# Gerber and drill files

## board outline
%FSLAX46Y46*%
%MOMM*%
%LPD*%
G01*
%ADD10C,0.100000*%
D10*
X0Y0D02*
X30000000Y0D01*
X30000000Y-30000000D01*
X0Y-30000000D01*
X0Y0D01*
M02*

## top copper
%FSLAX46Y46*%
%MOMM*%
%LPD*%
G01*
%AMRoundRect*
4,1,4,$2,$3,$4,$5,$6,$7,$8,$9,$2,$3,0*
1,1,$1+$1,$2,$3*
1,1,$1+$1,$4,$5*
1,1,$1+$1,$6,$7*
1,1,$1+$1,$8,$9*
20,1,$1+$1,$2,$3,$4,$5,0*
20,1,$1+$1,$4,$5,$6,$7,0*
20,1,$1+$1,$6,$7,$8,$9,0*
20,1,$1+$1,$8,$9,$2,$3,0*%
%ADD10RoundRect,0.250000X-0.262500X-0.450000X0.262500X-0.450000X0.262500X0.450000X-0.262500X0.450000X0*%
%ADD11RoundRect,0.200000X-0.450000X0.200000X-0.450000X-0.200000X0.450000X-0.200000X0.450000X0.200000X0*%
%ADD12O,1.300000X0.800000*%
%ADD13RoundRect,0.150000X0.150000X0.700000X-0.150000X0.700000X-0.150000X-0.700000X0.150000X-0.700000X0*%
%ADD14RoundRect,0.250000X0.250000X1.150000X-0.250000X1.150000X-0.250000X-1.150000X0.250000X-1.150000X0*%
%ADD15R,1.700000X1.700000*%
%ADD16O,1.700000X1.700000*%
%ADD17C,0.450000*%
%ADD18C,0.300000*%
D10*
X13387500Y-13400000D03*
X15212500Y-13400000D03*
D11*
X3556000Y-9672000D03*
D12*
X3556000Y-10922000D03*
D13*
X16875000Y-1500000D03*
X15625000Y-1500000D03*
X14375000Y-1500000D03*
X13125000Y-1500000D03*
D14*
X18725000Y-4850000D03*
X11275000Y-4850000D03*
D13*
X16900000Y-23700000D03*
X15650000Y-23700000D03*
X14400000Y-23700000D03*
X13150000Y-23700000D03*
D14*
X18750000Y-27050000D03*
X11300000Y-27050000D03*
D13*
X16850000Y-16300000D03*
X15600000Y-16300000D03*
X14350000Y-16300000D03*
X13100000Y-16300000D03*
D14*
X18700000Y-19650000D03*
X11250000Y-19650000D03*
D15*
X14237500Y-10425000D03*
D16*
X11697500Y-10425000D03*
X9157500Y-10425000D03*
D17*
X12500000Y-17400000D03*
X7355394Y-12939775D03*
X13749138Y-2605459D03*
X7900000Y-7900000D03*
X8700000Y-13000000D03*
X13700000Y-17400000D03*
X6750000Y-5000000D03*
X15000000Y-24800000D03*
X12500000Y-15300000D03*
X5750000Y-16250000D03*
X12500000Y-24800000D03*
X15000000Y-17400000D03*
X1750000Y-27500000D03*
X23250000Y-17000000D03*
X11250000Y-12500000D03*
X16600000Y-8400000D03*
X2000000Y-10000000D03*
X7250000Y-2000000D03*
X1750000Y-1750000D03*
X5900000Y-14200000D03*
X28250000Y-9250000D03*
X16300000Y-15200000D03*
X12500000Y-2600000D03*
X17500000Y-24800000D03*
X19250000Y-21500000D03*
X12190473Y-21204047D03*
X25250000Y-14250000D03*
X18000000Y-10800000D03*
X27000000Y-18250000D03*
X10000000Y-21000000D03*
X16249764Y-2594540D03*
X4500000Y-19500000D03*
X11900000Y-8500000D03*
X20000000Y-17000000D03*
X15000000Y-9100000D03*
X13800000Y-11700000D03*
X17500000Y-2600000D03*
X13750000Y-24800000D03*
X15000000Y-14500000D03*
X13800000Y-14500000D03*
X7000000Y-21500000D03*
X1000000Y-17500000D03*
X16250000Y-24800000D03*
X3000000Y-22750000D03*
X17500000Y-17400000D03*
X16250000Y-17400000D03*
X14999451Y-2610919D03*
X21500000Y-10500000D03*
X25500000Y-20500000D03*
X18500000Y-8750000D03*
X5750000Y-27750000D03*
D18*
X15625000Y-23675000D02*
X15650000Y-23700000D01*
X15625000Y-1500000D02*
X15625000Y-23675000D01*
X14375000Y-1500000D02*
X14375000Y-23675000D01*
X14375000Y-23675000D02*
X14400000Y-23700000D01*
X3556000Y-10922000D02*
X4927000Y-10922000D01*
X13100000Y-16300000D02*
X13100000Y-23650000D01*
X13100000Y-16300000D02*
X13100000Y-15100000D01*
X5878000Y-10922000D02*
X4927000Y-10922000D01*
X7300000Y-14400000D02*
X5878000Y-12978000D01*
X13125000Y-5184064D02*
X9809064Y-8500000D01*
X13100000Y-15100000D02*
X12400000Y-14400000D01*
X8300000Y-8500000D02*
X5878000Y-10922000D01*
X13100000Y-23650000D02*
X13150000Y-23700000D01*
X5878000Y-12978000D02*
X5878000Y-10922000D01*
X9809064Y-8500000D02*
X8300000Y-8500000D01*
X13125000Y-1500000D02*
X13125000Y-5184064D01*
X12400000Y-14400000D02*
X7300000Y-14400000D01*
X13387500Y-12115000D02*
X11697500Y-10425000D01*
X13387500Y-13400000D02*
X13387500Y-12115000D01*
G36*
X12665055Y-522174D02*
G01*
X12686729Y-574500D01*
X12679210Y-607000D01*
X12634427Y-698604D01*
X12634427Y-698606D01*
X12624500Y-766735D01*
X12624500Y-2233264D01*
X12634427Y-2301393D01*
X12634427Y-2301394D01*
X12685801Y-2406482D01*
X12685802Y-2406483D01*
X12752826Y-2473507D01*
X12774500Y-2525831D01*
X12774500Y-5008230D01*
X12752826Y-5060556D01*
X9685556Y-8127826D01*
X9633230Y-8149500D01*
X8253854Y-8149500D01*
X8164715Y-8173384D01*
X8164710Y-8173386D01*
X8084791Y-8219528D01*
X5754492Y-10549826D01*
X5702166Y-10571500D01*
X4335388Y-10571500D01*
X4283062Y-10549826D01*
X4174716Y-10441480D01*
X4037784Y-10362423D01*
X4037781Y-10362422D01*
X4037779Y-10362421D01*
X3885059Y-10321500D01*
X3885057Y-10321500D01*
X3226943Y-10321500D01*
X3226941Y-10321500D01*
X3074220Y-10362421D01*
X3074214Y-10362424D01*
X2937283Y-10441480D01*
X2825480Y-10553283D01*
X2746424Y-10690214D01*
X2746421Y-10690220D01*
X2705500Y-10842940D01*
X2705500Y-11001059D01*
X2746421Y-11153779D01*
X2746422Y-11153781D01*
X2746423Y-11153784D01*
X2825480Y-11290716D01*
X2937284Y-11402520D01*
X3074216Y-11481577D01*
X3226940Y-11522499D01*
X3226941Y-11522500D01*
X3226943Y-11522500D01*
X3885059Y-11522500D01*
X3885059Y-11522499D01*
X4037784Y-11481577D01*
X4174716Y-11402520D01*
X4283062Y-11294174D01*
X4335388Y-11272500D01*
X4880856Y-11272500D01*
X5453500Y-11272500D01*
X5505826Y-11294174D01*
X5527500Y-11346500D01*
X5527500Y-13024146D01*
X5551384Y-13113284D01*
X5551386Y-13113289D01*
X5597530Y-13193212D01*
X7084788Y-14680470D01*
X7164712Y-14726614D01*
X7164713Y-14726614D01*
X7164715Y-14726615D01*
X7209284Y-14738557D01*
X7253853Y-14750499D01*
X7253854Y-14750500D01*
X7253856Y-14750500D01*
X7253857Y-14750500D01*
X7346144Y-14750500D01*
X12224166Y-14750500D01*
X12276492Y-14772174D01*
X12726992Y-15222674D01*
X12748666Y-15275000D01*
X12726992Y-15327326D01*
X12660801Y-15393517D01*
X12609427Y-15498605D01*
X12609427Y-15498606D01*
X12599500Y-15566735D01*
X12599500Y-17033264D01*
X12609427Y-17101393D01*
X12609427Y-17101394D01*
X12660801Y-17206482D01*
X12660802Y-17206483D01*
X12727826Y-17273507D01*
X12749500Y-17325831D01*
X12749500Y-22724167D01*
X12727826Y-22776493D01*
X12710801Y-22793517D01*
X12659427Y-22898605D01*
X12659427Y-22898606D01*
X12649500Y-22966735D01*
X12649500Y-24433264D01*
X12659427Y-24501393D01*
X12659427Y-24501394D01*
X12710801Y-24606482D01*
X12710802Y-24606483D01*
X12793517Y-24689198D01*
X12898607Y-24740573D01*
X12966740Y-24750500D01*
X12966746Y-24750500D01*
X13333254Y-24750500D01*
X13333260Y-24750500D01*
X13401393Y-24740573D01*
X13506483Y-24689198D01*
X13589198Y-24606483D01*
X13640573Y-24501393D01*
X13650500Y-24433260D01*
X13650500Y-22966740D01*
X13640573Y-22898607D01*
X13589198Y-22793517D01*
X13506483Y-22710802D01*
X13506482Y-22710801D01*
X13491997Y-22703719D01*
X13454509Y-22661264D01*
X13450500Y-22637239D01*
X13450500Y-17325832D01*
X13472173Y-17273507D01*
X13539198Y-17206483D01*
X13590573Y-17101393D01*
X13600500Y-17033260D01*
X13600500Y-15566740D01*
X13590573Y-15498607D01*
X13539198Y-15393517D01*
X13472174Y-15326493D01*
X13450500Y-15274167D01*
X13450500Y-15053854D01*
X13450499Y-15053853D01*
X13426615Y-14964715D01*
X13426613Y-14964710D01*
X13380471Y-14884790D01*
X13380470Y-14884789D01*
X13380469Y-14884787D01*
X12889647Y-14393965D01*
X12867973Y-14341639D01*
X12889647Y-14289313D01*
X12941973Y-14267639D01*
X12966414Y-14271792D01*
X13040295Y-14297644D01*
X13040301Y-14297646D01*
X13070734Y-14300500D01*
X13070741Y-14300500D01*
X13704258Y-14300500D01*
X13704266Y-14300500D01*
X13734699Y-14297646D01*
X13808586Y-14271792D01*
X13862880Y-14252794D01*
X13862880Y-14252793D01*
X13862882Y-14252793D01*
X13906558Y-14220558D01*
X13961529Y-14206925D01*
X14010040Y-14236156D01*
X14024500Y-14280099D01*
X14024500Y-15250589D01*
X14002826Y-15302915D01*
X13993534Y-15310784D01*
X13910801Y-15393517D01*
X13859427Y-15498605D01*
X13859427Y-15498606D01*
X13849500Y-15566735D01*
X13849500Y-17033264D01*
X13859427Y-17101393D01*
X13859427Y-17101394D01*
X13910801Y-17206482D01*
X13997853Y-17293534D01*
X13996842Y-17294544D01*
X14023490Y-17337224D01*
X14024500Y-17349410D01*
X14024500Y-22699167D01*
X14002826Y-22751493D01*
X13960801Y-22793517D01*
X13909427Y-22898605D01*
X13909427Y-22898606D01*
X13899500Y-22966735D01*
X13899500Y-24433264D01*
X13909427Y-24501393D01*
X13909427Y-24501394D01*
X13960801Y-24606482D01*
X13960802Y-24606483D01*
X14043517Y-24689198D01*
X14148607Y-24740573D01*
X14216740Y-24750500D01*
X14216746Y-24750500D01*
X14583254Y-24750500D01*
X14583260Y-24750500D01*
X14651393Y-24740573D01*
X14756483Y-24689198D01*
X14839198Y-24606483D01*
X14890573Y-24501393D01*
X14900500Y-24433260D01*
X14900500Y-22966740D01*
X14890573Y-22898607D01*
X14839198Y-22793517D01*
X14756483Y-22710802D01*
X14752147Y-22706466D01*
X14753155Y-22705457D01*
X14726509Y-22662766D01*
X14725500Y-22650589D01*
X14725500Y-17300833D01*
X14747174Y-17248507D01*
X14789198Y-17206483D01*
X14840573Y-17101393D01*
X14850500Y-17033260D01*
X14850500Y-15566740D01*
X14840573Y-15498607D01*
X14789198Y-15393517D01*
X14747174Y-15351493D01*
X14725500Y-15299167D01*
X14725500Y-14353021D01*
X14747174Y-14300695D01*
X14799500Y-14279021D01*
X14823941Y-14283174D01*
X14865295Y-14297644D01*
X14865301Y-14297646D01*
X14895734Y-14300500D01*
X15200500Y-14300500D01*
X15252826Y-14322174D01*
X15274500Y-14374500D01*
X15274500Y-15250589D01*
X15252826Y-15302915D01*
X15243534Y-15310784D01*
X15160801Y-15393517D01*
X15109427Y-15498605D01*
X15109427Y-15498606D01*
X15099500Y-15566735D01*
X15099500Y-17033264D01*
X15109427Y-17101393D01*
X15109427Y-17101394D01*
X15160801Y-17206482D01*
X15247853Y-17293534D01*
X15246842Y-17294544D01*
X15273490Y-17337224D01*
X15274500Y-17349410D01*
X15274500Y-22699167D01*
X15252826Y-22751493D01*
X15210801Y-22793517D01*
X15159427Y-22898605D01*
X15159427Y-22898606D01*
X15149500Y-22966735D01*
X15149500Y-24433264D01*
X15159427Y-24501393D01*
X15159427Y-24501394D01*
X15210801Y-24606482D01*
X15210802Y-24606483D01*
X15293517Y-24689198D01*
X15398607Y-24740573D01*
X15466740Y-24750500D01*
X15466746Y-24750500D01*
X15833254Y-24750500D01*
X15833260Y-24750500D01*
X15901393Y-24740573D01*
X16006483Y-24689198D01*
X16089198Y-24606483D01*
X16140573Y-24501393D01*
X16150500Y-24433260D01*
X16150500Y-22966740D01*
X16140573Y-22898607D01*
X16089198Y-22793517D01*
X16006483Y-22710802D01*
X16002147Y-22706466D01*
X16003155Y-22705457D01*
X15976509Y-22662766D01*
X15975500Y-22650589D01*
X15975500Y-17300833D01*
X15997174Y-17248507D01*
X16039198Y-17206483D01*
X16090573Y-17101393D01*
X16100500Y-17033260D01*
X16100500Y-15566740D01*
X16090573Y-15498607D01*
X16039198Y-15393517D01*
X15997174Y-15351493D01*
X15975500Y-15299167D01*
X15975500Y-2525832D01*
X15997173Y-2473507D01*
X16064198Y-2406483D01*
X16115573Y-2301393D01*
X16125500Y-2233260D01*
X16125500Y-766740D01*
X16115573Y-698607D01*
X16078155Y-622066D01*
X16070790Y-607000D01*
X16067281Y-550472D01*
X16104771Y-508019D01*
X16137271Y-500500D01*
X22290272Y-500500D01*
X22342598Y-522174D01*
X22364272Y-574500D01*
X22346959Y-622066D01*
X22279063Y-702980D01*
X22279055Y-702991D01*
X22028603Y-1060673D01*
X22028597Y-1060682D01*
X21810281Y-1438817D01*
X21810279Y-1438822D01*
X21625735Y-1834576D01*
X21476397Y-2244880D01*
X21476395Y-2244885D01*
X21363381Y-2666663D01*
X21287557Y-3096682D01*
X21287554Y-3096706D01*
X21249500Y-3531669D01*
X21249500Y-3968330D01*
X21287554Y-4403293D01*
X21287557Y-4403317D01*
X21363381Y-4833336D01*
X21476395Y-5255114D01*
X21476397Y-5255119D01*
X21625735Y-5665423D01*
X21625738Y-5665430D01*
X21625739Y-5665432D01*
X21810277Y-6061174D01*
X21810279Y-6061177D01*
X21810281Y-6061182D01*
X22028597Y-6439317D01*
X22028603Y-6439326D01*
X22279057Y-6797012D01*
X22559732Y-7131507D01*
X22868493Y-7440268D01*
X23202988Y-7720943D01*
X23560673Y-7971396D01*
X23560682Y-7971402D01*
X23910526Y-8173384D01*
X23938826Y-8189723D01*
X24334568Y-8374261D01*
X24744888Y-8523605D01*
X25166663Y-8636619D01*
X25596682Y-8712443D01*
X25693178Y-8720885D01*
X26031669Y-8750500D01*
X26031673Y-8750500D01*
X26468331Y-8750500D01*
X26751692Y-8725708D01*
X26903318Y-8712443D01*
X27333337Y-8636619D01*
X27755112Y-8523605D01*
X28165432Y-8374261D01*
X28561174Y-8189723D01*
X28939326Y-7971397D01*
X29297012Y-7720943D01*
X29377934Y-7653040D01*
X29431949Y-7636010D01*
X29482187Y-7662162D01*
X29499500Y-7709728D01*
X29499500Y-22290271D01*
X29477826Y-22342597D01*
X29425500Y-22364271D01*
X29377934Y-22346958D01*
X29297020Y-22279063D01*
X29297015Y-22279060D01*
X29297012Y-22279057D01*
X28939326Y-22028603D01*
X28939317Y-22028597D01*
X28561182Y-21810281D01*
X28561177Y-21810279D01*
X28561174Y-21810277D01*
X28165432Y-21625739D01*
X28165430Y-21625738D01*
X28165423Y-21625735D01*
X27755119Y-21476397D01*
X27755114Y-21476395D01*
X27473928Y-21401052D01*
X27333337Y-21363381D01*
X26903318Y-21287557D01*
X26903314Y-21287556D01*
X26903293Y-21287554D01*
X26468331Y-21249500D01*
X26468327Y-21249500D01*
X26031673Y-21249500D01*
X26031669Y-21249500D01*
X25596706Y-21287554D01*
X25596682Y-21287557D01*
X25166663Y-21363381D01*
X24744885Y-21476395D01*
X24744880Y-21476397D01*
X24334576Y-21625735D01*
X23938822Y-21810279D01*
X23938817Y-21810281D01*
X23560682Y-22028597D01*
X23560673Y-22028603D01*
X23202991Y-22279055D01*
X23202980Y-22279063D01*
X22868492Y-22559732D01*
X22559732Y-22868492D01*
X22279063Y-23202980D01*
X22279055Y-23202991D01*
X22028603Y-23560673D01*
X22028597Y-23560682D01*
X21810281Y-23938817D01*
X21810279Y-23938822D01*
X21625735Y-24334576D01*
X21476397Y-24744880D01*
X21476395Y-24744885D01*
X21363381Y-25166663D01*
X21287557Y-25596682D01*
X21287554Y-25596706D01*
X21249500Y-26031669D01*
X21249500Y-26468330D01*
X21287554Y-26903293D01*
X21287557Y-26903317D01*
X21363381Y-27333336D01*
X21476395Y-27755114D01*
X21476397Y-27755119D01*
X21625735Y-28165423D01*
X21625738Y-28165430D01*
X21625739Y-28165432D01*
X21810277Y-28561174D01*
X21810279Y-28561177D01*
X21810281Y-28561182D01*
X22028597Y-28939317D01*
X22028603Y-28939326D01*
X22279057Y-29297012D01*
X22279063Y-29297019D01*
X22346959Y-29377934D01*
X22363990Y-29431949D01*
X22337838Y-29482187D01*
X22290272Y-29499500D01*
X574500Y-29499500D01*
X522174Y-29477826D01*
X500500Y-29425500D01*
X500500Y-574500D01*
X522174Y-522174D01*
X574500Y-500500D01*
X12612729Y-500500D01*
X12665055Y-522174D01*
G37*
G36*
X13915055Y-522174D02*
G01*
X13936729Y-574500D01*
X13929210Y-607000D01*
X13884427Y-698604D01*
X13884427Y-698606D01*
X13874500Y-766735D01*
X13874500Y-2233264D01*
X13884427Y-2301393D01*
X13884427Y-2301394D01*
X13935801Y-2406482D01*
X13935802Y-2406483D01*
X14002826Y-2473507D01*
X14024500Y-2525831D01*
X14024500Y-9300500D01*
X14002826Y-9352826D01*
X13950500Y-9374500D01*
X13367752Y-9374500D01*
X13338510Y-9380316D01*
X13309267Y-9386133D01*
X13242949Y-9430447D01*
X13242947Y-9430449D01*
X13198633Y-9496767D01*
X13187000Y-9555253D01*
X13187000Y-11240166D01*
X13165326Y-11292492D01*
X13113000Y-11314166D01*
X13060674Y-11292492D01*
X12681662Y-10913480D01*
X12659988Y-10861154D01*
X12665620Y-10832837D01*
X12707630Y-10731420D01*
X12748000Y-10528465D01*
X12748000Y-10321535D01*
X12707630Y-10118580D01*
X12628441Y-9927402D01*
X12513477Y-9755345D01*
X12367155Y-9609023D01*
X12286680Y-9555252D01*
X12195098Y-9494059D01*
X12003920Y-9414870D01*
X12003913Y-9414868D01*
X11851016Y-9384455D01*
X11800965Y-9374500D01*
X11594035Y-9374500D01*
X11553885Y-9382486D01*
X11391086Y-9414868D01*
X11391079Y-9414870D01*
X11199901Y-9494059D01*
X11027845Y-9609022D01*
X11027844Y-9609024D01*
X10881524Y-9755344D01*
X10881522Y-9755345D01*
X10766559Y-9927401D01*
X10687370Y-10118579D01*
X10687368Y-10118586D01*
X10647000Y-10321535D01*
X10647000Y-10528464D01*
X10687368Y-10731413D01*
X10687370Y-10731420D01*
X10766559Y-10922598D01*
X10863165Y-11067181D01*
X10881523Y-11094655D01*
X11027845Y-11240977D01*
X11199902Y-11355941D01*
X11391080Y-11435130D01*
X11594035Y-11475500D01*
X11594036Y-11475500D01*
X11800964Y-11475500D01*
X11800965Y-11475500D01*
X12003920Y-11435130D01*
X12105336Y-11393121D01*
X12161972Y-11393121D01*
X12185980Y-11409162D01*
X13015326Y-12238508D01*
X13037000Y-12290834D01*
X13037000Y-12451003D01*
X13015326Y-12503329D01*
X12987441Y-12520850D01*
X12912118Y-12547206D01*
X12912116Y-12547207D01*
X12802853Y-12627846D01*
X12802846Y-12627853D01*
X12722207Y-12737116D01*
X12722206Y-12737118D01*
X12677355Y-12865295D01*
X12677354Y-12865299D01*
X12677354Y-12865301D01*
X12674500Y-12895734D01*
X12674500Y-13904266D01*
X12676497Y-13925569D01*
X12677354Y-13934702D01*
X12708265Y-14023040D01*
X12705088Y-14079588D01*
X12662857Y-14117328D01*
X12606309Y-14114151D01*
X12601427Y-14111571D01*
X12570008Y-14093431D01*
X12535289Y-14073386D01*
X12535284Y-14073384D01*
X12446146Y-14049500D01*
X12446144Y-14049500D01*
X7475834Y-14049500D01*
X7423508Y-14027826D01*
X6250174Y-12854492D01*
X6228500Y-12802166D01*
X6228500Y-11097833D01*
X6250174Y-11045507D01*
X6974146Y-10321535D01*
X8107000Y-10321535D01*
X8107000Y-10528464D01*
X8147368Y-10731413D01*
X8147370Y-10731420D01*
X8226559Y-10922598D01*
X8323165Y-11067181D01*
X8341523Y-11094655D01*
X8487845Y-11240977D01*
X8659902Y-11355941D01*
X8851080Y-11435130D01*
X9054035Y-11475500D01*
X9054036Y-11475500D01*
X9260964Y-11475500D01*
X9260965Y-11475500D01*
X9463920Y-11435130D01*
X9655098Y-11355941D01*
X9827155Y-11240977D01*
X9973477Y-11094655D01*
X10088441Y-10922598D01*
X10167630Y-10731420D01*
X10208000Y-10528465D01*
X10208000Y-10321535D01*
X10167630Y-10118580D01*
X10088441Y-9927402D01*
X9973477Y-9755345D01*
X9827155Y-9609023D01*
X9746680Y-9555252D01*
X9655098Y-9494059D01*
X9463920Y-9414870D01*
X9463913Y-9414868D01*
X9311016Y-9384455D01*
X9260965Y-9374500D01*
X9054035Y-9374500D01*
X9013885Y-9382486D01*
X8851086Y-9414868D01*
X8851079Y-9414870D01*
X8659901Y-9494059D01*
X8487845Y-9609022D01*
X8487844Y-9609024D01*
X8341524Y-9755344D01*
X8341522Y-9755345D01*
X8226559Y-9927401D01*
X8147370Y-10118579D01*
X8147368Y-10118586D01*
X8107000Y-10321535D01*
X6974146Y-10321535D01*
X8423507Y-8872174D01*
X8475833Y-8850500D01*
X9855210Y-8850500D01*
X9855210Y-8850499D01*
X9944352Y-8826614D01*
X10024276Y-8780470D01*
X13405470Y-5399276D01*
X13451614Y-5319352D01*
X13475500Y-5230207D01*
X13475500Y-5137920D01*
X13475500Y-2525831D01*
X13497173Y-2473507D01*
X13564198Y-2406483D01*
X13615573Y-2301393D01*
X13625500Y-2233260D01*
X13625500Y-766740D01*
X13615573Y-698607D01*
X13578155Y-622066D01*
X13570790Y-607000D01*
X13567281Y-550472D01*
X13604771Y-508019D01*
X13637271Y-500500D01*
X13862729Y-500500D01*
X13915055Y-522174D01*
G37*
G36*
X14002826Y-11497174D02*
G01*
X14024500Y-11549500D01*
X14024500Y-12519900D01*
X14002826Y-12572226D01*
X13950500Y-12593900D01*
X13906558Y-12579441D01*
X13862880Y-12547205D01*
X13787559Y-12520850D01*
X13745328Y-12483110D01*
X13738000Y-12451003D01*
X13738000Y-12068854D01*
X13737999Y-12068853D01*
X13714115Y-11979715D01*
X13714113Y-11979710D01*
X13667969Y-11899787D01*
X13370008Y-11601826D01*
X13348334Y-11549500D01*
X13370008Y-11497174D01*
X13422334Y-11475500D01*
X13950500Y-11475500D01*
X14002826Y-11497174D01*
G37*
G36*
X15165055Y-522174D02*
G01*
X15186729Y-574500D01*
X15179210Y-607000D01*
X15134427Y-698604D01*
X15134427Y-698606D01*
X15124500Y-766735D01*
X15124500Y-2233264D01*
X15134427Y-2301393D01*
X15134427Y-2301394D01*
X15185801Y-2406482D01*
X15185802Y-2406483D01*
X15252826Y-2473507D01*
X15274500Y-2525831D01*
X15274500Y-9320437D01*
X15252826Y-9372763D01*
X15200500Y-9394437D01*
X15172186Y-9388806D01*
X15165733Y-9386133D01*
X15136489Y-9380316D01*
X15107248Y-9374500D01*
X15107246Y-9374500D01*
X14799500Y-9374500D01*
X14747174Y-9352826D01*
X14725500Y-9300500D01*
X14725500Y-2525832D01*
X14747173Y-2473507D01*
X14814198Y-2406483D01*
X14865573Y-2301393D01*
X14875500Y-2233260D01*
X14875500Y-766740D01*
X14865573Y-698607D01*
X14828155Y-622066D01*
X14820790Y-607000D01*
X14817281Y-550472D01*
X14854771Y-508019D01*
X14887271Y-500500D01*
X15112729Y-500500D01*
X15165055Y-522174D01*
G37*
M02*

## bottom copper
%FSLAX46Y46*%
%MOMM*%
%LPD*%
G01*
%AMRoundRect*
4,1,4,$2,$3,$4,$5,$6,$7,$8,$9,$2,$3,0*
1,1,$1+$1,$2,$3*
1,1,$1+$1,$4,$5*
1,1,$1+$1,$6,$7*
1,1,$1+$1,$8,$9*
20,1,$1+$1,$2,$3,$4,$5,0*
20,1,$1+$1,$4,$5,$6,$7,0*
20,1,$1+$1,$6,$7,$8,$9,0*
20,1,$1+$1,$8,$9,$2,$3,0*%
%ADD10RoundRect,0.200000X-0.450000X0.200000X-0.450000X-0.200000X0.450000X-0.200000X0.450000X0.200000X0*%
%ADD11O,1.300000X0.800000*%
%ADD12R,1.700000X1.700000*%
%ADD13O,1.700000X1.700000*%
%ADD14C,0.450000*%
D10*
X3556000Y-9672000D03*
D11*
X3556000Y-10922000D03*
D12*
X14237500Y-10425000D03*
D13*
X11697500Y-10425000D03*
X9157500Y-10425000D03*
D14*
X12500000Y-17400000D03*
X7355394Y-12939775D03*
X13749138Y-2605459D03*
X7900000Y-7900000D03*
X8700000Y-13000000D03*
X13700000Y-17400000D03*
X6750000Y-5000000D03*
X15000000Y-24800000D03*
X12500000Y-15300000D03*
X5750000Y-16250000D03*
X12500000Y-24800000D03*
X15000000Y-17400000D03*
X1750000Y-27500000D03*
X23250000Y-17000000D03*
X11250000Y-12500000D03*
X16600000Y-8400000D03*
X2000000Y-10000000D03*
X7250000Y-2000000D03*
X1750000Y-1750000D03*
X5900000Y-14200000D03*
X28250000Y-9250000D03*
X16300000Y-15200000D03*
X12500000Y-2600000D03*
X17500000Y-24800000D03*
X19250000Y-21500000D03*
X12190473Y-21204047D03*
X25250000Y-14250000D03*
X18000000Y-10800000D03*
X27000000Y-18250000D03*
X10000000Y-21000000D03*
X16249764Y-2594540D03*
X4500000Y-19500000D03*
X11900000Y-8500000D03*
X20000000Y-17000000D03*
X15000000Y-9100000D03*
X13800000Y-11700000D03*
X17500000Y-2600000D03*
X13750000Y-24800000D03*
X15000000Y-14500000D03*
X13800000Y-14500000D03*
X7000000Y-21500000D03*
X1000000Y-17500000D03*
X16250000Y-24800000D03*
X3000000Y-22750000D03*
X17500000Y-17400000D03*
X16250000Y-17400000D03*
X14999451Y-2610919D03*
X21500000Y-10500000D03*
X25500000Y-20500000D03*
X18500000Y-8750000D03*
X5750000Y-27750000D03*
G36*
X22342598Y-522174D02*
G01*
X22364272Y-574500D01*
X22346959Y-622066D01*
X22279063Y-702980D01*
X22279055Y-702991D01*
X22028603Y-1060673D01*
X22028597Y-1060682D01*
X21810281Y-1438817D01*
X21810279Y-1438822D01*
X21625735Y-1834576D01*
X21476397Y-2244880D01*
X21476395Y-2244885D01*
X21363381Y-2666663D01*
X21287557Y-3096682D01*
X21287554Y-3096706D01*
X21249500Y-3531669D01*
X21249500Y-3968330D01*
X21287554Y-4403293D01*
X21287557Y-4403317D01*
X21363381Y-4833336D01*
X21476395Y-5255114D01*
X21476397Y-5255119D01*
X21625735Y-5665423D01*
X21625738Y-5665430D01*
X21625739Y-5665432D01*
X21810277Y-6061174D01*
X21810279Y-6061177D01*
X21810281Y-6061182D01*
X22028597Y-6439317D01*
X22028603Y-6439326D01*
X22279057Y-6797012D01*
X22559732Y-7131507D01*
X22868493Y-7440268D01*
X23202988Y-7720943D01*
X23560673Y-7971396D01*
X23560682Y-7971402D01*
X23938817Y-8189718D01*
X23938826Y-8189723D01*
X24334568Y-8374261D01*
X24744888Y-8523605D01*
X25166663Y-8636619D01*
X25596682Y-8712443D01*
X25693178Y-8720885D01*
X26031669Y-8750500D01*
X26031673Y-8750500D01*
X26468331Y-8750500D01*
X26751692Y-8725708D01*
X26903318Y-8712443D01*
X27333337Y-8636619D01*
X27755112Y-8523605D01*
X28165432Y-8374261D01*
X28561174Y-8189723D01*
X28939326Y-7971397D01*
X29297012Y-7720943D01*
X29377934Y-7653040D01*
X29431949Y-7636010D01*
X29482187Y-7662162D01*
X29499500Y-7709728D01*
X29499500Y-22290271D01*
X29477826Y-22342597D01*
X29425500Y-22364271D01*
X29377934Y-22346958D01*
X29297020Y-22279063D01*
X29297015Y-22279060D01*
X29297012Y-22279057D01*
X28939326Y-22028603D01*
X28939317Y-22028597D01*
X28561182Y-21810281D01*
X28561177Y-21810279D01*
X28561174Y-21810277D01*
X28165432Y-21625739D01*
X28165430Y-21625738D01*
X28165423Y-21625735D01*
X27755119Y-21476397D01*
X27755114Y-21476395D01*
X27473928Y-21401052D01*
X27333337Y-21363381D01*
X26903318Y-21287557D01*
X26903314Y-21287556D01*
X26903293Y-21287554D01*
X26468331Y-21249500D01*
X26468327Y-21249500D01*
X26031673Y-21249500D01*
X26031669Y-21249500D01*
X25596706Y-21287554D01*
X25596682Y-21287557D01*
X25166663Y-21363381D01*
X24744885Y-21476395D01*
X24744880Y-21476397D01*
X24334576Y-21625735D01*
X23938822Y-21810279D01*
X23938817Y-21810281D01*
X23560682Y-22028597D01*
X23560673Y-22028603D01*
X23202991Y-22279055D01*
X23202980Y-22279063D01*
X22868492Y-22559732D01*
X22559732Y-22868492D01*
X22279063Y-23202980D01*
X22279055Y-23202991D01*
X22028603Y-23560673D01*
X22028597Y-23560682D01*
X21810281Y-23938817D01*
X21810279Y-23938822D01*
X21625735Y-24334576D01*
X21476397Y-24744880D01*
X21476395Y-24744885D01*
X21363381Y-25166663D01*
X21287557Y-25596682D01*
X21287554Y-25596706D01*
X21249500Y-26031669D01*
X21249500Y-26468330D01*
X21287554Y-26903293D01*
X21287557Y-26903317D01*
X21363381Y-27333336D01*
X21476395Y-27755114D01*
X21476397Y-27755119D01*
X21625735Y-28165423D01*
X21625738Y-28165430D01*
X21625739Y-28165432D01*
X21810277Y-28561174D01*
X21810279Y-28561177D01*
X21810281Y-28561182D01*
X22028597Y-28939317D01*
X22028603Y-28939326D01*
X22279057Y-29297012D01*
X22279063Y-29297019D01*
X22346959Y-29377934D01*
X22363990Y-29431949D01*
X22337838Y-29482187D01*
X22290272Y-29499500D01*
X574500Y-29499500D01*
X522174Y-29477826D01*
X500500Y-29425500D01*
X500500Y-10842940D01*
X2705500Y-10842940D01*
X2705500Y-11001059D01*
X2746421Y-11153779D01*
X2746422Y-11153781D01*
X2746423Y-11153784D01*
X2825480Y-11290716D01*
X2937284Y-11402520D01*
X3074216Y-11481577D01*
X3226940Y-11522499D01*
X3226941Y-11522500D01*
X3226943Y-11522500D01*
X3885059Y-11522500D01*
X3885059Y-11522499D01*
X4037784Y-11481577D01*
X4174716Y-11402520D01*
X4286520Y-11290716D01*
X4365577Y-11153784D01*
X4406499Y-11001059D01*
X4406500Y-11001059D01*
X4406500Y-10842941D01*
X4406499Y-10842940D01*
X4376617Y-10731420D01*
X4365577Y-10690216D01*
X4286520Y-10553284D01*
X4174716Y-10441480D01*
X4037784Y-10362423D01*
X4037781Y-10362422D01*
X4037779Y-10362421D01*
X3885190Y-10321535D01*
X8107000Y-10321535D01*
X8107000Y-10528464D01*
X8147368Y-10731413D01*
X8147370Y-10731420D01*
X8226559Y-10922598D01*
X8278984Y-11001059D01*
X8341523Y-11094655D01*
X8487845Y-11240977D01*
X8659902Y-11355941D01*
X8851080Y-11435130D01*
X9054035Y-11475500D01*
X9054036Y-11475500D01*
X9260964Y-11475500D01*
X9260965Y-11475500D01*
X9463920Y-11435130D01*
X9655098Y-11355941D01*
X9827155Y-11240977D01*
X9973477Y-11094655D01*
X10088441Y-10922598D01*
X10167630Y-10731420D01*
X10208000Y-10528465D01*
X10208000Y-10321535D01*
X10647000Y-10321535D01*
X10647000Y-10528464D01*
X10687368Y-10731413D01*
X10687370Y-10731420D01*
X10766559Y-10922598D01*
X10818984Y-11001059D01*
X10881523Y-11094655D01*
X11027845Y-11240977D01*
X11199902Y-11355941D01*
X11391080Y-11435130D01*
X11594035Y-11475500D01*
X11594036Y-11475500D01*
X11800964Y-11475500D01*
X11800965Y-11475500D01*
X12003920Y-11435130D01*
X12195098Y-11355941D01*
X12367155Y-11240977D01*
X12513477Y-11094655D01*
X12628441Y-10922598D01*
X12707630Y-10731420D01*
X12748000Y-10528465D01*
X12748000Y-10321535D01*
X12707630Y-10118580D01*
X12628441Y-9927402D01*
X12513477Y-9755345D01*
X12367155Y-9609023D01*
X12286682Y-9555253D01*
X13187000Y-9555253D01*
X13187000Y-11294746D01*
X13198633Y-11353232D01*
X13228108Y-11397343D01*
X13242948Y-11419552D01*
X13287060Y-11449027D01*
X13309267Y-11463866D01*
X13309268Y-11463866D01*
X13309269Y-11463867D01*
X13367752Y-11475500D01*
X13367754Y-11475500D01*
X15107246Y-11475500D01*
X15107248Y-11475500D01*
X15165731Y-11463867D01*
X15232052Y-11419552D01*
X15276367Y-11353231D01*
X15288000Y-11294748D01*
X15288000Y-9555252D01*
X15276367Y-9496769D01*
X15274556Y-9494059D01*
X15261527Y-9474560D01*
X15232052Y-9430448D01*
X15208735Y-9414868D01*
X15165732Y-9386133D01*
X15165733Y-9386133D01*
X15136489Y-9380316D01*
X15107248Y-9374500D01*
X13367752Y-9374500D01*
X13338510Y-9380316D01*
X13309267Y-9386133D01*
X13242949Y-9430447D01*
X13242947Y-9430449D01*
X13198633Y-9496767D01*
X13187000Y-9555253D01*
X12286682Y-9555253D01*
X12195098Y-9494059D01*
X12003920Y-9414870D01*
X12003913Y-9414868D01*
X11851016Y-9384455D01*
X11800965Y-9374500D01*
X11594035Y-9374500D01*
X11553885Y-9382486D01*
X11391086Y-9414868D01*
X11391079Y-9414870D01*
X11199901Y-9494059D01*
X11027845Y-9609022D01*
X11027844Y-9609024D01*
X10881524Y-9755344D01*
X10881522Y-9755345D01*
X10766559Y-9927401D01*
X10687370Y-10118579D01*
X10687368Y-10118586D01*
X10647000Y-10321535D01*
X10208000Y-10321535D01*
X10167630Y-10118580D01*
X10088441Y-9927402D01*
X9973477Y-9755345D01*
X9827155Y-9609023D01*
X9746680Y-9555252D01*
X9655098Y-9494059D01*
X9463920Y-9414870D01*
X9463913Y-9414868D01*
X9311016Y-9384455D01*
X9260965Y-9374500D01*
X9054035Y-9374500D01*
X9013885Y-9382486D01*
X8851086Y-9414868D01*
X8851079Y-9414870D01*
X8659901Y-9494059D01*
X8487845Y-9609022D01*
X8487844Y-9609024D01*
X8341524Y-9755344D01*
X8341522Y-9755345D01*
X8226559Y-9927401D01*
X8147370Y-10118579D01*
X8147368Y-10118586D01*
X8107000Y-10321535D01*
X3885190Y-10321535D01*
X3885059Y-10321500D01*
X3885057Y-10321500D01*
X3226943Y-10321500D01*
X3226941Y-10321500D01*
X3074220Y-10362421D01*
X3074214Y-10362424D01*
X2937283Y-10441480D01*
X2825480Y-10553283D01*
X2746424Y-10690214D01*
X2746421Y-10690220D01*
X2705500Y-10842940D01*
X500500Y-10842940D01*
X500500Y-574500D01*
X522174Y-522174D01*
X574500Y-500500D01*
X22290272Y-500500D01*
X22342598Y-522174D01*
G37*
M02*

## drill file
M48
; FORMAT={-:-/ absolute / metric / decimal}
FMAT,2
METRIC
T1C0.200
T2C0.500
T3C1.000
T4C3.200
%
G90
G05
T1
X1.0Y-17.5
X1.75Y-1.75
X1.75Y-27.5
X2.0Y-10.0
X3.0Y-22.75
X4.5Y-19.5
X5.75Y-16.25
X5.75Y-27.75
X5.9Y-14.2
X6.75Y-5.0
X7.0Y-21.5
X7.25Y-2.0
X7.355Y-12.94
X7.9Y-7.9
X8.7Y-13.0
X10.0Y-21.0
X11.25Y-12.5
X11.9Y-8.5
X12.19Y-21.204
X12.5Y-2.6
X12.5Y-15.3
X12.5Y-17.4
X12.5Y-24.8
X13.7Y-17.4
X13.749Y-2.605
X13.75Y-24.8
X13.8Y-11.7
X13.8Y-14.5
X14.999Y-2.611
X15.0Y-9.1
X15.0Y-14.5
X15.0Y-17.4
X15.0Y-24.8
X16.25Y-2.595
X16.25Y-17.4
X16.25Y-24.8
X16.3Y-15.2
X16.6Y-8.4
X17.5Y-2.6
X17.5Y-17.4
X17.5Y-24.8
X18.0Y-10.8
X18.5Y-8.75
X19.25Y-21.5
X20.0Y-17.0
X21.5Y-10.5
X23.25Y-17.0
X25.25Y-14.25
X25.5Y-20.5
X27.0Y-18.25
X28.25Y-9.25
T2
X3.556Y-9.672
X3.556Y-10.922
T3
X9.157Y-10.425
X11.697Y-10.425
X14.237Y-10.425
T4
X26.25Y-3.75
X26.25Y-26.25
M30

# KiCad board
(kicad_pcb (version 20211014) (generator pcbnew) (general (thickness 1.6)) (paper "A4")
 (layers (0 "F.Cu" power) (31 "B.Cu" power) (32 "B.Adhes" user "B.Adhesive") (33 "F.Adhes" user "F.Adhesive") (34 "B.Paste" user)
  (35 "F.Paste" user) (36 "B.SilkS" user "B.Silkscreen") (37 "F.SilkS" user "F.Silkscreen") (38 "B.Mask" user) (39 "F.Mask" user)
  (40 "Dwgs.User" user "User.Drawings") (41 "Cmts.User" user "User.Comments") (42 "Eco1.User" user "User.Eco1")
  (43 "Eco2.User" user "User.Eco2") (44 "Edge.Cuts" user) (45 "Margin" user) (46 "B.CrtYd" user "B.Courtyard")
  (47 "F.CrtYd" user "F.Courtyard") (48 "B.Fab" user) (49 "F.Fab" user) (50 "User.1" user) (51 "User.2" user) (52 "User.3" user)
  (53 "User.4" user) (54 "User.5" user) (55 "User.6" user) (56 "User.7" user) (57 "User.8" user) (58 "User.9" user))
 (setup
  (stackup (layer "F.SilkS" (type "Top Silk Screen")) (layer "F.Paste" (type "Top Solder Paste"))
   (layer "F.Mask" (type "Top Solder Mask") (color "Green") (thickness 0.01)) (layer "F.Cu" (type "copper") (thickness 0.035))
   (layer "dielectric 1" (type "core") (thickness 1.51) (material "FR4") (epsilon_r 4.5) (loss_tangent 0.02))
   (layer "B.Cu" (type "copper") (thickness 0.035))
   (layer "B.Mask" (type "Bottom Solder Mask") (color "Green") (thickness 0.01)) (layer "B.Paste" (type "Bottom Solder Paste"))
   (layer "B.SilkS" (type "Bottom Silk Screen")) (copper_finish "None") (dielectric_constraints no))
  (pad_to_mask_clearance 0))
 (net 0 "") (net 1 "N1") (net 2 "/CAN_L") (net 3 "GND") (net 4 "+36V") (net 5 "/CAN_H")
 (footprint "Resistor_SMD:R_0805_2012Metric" (layer "F.Cu") (at 14.3 13.4)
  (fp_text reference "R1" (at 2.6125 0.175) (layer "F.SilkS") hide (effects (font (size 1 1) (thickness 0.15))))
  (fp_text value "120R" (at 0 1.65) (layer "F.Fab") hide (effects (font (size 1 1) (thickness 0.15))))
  (pad "1" smd roundrect locked (at -0.9125 0) (size 1.025 1.4) (layers "F.Cu" "F.Paste" "F.Mask") (roundrect_rratio 0.243902439)
   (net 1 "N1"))
  (pad "2" smd roundrect locked (at 0.9125 0) (size 1.025 1.4) (layers "F.Cu" "F.Paste" "F.Mask") (roundrect_rratio 0.243902439)
   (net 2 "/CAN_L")))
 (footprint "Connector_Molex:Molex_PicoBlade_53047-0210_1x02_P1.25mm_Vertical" (layer "F.Cu") (at 3.556 9.672 -90)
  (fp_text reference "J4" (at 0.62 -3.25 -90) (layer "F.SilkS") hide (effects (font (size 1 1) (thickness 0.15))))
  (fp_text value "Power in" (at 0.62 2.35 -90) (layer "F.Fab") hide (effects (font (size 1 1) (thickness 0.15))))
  (pad "1" thru_hole roundrect locked (at 0 0 270) (size 0.8 1.3) (drill 0.5) (layers *.Cu *.Mask) (roundrect_rratio 0.25) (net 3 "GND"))
  (pad "2" thru_hole oval locked (at 1.25 0 270) (size 0.8 1.3) (drill 0.5) (layers *.Cu *.Mask) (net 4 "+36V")))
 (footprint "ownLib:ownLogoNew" (layer "F.Cu") (at 22.2 12.8 -90)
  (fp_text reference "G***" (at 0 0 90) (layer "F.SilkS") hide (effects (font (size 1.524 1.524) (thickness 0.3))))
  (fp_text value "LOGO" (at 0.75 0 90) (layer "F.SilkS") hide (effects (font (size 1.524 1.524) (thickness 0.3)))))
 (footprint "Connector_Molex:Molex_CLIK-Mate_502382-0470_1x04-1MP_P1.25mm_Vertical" (layer "F.Cu") (at 15 3.45 180)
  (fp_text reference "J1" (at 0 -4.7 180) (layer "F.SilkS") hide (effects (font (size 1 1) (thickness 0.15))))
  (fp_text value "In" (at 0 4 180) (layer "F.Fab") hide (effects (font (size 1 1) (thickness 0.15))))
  (pad "1" smd roundrect locked (at -1.875 1.95 180) (size 0.6 1.7) (layers "F.Cu" "F.Paste" "F.Mask") (roundrect_rratio 0.25) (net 3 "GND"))
  (pad "2" smd roundrect locked (at -0.625 1.95 180) (size 0.6 1.7) (layers "F.Cu" "F.Paste" "F.Mask") (roundrect_rratio 0.25)
   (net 2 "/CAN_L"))
  (pad "3" smd roundrect locked (at 0.625 1.95 180) (size 0.6 1.7) (layers "F.Cu" "F.Paste" "F.Mask") (roundrect_rratio 0.25)
   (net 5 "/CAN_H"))
  (pad "4" smd roundrect locked (at 1.875 1.95 180) (size 0.6 1.7) (layers "F.Cu" "F.Paste" "F.Mask") (roundrect_rratio 0.25) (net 4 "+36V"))
  (pad "MP" smd roundrect locked (at -3.725 -1.4 180) (size 1 2.8) (layers "F.Cu" "F.Paste" "F.Mask") (roundrect_rratio 0.25) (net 3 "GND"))
  (pad "MP" smd roundrect locked (at 3.725 -1.4 180) (size 1 2.8) (layers "F.Cu" "F.Paste" "F.Mask") (roundrect_rratio 0.25) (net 3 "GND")))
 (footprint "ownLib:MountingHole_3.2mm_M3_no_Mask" (layer "F.Cu") (at 26.25 26.25)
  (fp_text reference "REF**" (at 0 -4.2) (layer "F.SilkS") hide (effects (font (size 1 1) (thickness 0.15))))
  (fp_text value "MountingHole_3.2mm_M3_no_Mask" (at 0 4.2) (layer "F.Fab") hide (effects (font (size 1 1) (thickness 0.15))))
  (pad "" np_thru_hole circle locked (at 0 0) (size 3.2 3.2) (drill 3.2) (layers *.Cu *.Mask) (solder_mask_margin 1.9) (clearance 3.4)
   (zone_connect 0)))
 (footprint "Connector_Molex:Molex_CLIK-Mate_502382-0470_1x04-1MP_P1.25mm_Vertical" (layer "F.Cu") (at 15.025 25.65 180)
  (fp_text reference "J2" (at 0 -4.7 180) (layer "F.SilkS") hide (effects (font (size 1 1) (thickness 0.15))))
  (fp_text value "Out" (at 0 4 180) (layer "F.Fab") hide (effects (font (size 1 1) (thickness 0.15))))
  (pad "1" smd roundrect locked (at -1.875 1.95 180) (size 0.6 1.7) (layers "F.Cu" "F.Paste" "F.Mask") (roundrect_rratio 0.25) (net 3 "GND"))
  (pad "2" smd roundrect locked (at -0.625 1.95 180) (size 0.6 1.7) (layers "F.Cu" "F.Paste" "F.Mask") (roundrect_rratio 0.25)
   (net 2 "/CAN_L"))
  (pad "3" smd roundrect locked (at 0.625 1.95 180) (size 0.6 1.7) (layers "F.Cu" "F.Paste" "F.Mask") (roundrect_rratio 0.25)
   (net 5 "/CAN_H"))
  (pad "4" smd roundrect locked (at 1.875 1.95 180) (size 0.6 1.7) (layers "F.Cu" "F.Paste" "F.Mask") (roundrect_rratio 0.25) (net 4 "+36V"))
  (pad "MP" smd roundrect locked (at -3.725 -1.4 180) (size 1 2.8) (layers "F.Cu" "F.Paste" "F.Mask") (roundrect_rratio 0.25) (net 3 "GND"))
  (pad "MP" smd roundrect locked (at 3.725 -1.4 180) (size 1 2.8) (layers "F.Cu" "F.Paste" "F.Mask") (roundrect_rratio 0.25) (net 3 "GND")))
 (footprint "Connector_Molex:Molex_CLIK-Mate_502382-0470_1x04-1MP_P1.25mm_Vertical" (layer "F.Cu") (at 14.975 18.25 180)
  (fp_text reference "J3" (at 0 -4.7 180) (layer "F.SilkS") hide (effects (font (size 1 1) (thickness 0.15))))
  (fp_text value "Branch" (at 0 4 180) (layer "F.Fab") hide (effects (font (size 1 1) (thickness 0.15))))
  (pad "1" smd roundrect locked (at -1.875 1.95 180) (size 0.6 1.7) (layers "F.Cu" "F.Paste" "F.Mask") (roundrect_rratio 0.25) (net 3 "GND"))
  (pad "2" smd roundrect locked (at -0.625 1.95 180) (size 0.6 1.7) (layers "F.Cu" "F.Paste" "F.Mask") (roundrect_rratio 0.25)
   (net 2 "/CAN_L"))
  (pad "3" smd roundrect locked (at 0.625 1.95 180) (size 0.6 1.7) (layers "F.Cu" "F.Paste" "F.Mask") (roundrect_rratio 0.25)
   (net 5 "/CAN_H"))
  (pad "4" smd roundrect locked (at 1.875 1.95 180) (size 0.6 1.7) (layers "F.Cu" "F.Paste" "F.Mask") (roundrect_rratio 0.25) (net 4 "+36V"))
  (pad "MP" smd roundrect locked (at -3.725 -1.4 180) (size 1 2.8) (layers "F.Cu" "F.Paste" "F.Mask") (roundrect_rratio 0.25) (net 3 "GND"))
  (pad "MP" smd roundrect locked (at 3.725 -1.4 180) (size 1 2.8) (layers "F.Cu" "F.Paste" "F.Mask") (roundrect_rratio 0.25) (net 3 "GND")))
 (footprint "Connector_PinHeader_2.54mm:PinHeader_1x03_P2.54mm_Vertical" (layer "F.Cu") (at 14.2375 10.425 -90)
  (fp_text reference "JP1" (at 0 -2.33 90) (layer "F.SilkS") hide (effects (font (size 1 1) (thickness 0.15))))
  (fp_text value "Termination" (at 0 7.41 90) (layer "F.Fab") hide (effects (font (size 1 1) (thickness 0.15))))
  (pad "1" thru_hole rect locked (at 0 0 270) (size 1.7 1.7) (drill 1) (layers *.Cu *.Mask) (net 5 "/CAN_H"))
  (pad "2" thru_hole oval locked (at 0 2.54 270) (size 1.7 1.7) (drill 1) (layers *.Cu *.Mask) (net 1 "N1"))
  (pad "3" thru_hole oval locked (at 0 5.08 270) (size 1.7 1.7) (drill 1) (layers *.Cu *.Mask)))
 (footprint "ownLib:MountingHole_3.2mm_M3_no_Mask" (layer "F.Cu") (at 26.25 3.75)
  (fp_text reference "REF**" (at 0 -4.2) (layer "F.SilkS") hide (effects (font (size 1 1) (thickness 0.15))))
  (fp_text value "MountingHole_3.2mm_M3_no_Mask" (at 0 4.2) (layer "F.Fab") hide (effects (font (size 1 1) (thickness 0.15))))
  (pad "" np_thru_hole circle locked (at 0 0) (size 3.2 3.2) (drill 3.2) (layers *.Cu *.Mask) (solder_mask_margin 1.9) (clearance 3.4)
   (zone_connect 0)))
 (gr_rect (start 0 0) (end 30 30) (layer "Edge.Cuts") (width 0.1) (fill none))
 (via (at 12.5 17.4) (size 0.45) (drill 0.2) (layers "F.Cu" "B.Cu") (free) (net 3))
 (via (at 7.355394 12.939775) (size 0.45) (drill 0.2) (layers "F.Cu" "B.Cu") (free) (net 3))
 (via (at 13.749138 2.605459) (size 0.45) (drill 0.2) (layers "F.Cu" "B.Cu") (free) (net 3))
 (via (at 7.9 7.9) (size 0.45) (drill 0.2) (layers "F.Cu" "B.Cu") (free) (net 3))
 (via (at 8.7 13) (size 0.45) (drill 0.2) (layers "F.Cu" "B.Cu") (free) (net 3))
 (via (at 13.7 17.4) (size 0.45) (drill 0.2) (layers "F.Cu" "B.Cu") (free) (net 3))
 (via (at 6.75 5) (size 0.45) (drill 0.2) (layers "F.Cu" "B.Cu") (free) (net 3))
 (via (at 15 24.8) (size 0.45) (drill 0.2) (layers "F.Cu" "B.Cu") (free) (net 3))
 (via (at 12.5 15.3) (size 0.45) (drill 0.2) (layers "F.Cu" "B.Cu") (free) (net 3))
 (via (at 5.75 16.25) (size 0.45) (drill 0.2) (layers "F.Cu" "B.Cu") (free) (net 3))
 (via (at 12.5 24.8) (size 0.45) (drill 0.2) (layers "F.Cu" "B.Cu") (free) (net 3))
 (via (at 15 17.4) (size 0.45) (drill 0.2) (layers "F.Cu" "B.Cu") (free) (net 3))
 (via (at 1.75 27.5) (size 0.45) (drill 0.2) (layers "F.Cu" "B.Cu") (free) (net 3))
 (via (at 23.25 17) (size 0.45) (drill 0.2) (layers "F.Cu" "B.Cu") (free) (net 3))
 (via (at 11.25 12.5) (size 0.45) (drill 0.2) (layers "F.Cu" "B.Cu") (free) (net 3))
 (via (at 16.6 8.4) (size 0.45) (drill 0.2) (layers "F.Cu" "B.Cu") (free) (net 3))
 (via (at 2 10) (size 0.45) (drill 0.2) (layers "F.Cu" "B.Cu") (free) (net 3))
 (via (at 7.25 2) (size 0.45) (drill 0.2) (layers "F.Cu" "B.Cu") (free) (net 3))
 (via (at 1.75 1.75) (size 0.45) (drill 0.2) (layers "F.Cu" "B.Cu") (free) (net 3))
 (via (at 5.9 14.2) (size 0.45) (drill 0.2) (layers "F.Cu" "B.Cu") (free) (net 3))
 (via (at 28.25 9.25) (size 0.45) (drill 0.2) (layers "F.Cu" "B.Cu") (free) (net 3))
 (via (at 16.3 15.2) (size 0.45) (drill 0.2) (layers "F.Cu" "B.Cu") (free) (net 3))
 (via (at 12.5 2.6) (size 0.45) (drill 0.2) (layers "F.Cu" "B.Cu") (free) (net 3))
 (via (at 17.5 24.8) (size 0.45) (drill 0.2) (layers "F.Cu" "B.Cu") (free) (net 3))
 (via (at 19.25 21.5) (size 0.45) (drill 0.2) (layers "F.Cu" "B.Cu") (free) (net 3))
 (via (at 12.190473 21.204047) (size 0.45) (drill 0.2) (layers "F.Cu" "B.Cu") (free) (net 3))
 (via (at 25.25 14.25) (size 0.45) (drill 0.2) (layers "F.Cu" "B.Cu") (free) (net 3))
 (via (at 18 10.8) (size 0.45) (drill 0.2) (layers "F.Cu" "B.Cu") (free) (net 3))
 (via (at 27 18.25) (size 0.45) (drill 0.2) (layers "F.Cu" "B.Cu") (free) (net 3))
 (via (at 10 21) (size 0.45) (drill 0.2) (layers "F.Cu" "B.Cu") (free) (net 3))
 (via (at 16.249764 2.59454) (size 0.45) (drill 0.2) (layers "F.Cu" "B.Cu") (free) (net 3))
 (via (at 4.5 19.5) (size 0.45) (drill 0.2) (layers "F.Cu" "B.Cu") (free) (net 3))
 (via (at 11.9 8.5) (size 0.45) (drill 0.2) (layers "F.Cu" "B.Cu") (free) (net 3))
 (via (at 20 17) (size 0.45) (drill 0.2) (layers "F.Cu" "B.Cu") (free) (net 3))
 (via (at 15 9.1) (size 0.45) (drill 0.2) (layers "F.Cu" "B.Cu") (free) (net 3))
 (via (at 13.8 11.7) (size 0.45) (drill 0.2) (layers "F.Cu" "B.Cu") (free) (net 3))
 (via (at 17.5 2.6) (size 0.45) (drill 0.2) (layers "F.Cu" "B.Cu") (free) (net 3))
 (via (at 13.75 24.8) (size 0.45) (drill 0.2) (layers "F.Cu" "B.Cu") (free) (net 3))
 (via (at 15 14.5) (size 0.45) (drill 0.2) (layers "F.Cu" "B.Cu") (free) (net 3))
 (via (at 13.8 14.5) (size 0.45) (drill 0.2) (layers "F.Cu" "B.Cu") (free) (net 3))
 (via (at 7 21.5) (size 0.45) (drill 0.2) (layers "F.Cu" "B.Cu") (free) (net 3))
 (via (at 1 17.5) (size 0.45) (drill 0.2) (layers "F.Cu" "B.Cu") (free) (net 3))
 (via (at 16.25 24.8) (size 0.45) (drill 0.2) (layers "F.Cu" "B.Cu") (free) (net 3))
 (via (at 3 22.75) (size 0.45) (drill 0.2) (layers "F.Cu" "B.Cu") (free) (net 3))
 (via (at 17.5 17.4) (size 0.45) (drill 0.2) (layers "F.Cu" "B.Cu") (free) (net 3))
 (via (at 16.25 17.4) (size 0.45) (drill 0.2) (layers "F.Cu" "B.Cu") (free) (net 3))
 (via (at 14.999451 2.610919) (size 0.45) (drill 0.2) (layers "F.Cu" "B.Cu") (free) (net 3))
 (via (at 21.5 10.5) (size 0.45) (drill 0.2) (layers "F.Cu" "B.Cu") (free) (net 3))
 (via (at 25.5 20.5) (size 0.45) (drill 0.2) (layers "F.Cu" "B.Cu") (free) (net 3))
 (via (at 18.5 8.75) (size 0.45) (drill 0.2) (layers "F.Cu" "B.Cu") (free) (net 3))
 (via (at 5.75 27.75) (size 0.45) (drill 0.2) (layers "F.Cu" "B.Cu") (free) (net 3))
 (segment (start 15.625 23.675) (end 15.65 23.7) (width 0.3) (layer "F.Cu") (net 2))
 (segment (start 15.625 1.5) (end 15.625 23.675) (width 0.3) (layer "F.Cu") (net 2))
 (segment (start 14.375 1.5) (end 14.375 23.675) (width 0.3) (layer "F.Cu") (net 5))
 (segment (start 14.375 23.675) (end 14.4 23.7) (width 0.3) (layer "F.Cu") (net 5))
 (segment (start 3.556 10.922) (end 4.927 10.922) (width 0.3) (layer "F.Cu") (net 4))
 (segment (start 13.1 16.3) (end 13.1 23.65) (width 0.3) (layer "F.Cu") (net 4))
 (segment (start 13.1 16.3) (end 13.1 15.1) (width 0.3) (layer "F.Cu") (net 4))
 (segment (start 5.878 10.922) (end 4.927 10.922) (width 0.3) (layer "F.Cu") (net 4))
 (segment (start 7.3 14.4) (end 5.878 12.978) (width 0.3) (layer "F.Cu") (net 4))
 (segment (start 13.125 5.184064) (end 9.809064 8.5) (width 0.3) (layer "F.Cu") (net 4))
 (segment (start 13.1 15.1) (end 12.4 14.4) (width 0.3) (layer "F.Cu") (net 4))
 (segment (start 8.3 8.5) (end 5.878 10.922) (width 0.3) (layer "F.Cu") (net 4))
 (segment (start 13.1 23.65) (end 13.15 23.7) (width 0.3) (layer "F.Cu") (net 4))
 (segment (start 5.878 12.978) (end 5.878 10.922) (width 0.3) (layer "F.Cu") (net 4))
 (segment (start 9.809064 8.5) (end 8.3 8.5) (width 0.3) (layer "F.Cu") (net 4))
 (segment (start 13.125 1.5) (end 13.125 5.184064) (width 0.3) (layer "F.Cu") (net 4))
 (segment (start 12.4 14.4) (end 7.3 14.4) (width 0.3) (layer "F.Cu") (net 4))
 (segment (start 13.3875 12.115) (end 11.6975 10.425) (width 0.3) (layer "F.Cu") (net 1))
 (segment (start 13.3875 13.4) (end 13.3875 12.115) (width 0.3) (layer "F.Cu") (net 1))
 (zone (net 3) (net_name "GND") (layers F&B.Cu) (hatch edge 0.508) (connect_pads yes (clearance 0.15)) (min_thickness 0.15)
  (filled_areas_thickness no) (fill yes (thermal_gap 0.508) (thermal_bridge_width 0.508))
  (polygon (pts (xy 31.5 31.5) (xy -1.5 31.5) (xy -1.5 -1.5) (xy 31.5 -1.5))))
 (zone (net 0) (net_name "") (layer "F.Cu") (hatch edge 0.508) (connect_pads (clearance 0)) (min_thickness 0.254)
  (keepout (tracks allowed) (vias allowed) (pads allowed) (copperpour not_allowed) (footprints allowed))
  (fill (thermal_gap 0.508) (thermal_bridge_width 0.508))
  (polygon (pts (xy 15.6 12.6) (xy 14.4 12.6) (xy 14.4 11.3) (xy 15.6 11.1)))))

